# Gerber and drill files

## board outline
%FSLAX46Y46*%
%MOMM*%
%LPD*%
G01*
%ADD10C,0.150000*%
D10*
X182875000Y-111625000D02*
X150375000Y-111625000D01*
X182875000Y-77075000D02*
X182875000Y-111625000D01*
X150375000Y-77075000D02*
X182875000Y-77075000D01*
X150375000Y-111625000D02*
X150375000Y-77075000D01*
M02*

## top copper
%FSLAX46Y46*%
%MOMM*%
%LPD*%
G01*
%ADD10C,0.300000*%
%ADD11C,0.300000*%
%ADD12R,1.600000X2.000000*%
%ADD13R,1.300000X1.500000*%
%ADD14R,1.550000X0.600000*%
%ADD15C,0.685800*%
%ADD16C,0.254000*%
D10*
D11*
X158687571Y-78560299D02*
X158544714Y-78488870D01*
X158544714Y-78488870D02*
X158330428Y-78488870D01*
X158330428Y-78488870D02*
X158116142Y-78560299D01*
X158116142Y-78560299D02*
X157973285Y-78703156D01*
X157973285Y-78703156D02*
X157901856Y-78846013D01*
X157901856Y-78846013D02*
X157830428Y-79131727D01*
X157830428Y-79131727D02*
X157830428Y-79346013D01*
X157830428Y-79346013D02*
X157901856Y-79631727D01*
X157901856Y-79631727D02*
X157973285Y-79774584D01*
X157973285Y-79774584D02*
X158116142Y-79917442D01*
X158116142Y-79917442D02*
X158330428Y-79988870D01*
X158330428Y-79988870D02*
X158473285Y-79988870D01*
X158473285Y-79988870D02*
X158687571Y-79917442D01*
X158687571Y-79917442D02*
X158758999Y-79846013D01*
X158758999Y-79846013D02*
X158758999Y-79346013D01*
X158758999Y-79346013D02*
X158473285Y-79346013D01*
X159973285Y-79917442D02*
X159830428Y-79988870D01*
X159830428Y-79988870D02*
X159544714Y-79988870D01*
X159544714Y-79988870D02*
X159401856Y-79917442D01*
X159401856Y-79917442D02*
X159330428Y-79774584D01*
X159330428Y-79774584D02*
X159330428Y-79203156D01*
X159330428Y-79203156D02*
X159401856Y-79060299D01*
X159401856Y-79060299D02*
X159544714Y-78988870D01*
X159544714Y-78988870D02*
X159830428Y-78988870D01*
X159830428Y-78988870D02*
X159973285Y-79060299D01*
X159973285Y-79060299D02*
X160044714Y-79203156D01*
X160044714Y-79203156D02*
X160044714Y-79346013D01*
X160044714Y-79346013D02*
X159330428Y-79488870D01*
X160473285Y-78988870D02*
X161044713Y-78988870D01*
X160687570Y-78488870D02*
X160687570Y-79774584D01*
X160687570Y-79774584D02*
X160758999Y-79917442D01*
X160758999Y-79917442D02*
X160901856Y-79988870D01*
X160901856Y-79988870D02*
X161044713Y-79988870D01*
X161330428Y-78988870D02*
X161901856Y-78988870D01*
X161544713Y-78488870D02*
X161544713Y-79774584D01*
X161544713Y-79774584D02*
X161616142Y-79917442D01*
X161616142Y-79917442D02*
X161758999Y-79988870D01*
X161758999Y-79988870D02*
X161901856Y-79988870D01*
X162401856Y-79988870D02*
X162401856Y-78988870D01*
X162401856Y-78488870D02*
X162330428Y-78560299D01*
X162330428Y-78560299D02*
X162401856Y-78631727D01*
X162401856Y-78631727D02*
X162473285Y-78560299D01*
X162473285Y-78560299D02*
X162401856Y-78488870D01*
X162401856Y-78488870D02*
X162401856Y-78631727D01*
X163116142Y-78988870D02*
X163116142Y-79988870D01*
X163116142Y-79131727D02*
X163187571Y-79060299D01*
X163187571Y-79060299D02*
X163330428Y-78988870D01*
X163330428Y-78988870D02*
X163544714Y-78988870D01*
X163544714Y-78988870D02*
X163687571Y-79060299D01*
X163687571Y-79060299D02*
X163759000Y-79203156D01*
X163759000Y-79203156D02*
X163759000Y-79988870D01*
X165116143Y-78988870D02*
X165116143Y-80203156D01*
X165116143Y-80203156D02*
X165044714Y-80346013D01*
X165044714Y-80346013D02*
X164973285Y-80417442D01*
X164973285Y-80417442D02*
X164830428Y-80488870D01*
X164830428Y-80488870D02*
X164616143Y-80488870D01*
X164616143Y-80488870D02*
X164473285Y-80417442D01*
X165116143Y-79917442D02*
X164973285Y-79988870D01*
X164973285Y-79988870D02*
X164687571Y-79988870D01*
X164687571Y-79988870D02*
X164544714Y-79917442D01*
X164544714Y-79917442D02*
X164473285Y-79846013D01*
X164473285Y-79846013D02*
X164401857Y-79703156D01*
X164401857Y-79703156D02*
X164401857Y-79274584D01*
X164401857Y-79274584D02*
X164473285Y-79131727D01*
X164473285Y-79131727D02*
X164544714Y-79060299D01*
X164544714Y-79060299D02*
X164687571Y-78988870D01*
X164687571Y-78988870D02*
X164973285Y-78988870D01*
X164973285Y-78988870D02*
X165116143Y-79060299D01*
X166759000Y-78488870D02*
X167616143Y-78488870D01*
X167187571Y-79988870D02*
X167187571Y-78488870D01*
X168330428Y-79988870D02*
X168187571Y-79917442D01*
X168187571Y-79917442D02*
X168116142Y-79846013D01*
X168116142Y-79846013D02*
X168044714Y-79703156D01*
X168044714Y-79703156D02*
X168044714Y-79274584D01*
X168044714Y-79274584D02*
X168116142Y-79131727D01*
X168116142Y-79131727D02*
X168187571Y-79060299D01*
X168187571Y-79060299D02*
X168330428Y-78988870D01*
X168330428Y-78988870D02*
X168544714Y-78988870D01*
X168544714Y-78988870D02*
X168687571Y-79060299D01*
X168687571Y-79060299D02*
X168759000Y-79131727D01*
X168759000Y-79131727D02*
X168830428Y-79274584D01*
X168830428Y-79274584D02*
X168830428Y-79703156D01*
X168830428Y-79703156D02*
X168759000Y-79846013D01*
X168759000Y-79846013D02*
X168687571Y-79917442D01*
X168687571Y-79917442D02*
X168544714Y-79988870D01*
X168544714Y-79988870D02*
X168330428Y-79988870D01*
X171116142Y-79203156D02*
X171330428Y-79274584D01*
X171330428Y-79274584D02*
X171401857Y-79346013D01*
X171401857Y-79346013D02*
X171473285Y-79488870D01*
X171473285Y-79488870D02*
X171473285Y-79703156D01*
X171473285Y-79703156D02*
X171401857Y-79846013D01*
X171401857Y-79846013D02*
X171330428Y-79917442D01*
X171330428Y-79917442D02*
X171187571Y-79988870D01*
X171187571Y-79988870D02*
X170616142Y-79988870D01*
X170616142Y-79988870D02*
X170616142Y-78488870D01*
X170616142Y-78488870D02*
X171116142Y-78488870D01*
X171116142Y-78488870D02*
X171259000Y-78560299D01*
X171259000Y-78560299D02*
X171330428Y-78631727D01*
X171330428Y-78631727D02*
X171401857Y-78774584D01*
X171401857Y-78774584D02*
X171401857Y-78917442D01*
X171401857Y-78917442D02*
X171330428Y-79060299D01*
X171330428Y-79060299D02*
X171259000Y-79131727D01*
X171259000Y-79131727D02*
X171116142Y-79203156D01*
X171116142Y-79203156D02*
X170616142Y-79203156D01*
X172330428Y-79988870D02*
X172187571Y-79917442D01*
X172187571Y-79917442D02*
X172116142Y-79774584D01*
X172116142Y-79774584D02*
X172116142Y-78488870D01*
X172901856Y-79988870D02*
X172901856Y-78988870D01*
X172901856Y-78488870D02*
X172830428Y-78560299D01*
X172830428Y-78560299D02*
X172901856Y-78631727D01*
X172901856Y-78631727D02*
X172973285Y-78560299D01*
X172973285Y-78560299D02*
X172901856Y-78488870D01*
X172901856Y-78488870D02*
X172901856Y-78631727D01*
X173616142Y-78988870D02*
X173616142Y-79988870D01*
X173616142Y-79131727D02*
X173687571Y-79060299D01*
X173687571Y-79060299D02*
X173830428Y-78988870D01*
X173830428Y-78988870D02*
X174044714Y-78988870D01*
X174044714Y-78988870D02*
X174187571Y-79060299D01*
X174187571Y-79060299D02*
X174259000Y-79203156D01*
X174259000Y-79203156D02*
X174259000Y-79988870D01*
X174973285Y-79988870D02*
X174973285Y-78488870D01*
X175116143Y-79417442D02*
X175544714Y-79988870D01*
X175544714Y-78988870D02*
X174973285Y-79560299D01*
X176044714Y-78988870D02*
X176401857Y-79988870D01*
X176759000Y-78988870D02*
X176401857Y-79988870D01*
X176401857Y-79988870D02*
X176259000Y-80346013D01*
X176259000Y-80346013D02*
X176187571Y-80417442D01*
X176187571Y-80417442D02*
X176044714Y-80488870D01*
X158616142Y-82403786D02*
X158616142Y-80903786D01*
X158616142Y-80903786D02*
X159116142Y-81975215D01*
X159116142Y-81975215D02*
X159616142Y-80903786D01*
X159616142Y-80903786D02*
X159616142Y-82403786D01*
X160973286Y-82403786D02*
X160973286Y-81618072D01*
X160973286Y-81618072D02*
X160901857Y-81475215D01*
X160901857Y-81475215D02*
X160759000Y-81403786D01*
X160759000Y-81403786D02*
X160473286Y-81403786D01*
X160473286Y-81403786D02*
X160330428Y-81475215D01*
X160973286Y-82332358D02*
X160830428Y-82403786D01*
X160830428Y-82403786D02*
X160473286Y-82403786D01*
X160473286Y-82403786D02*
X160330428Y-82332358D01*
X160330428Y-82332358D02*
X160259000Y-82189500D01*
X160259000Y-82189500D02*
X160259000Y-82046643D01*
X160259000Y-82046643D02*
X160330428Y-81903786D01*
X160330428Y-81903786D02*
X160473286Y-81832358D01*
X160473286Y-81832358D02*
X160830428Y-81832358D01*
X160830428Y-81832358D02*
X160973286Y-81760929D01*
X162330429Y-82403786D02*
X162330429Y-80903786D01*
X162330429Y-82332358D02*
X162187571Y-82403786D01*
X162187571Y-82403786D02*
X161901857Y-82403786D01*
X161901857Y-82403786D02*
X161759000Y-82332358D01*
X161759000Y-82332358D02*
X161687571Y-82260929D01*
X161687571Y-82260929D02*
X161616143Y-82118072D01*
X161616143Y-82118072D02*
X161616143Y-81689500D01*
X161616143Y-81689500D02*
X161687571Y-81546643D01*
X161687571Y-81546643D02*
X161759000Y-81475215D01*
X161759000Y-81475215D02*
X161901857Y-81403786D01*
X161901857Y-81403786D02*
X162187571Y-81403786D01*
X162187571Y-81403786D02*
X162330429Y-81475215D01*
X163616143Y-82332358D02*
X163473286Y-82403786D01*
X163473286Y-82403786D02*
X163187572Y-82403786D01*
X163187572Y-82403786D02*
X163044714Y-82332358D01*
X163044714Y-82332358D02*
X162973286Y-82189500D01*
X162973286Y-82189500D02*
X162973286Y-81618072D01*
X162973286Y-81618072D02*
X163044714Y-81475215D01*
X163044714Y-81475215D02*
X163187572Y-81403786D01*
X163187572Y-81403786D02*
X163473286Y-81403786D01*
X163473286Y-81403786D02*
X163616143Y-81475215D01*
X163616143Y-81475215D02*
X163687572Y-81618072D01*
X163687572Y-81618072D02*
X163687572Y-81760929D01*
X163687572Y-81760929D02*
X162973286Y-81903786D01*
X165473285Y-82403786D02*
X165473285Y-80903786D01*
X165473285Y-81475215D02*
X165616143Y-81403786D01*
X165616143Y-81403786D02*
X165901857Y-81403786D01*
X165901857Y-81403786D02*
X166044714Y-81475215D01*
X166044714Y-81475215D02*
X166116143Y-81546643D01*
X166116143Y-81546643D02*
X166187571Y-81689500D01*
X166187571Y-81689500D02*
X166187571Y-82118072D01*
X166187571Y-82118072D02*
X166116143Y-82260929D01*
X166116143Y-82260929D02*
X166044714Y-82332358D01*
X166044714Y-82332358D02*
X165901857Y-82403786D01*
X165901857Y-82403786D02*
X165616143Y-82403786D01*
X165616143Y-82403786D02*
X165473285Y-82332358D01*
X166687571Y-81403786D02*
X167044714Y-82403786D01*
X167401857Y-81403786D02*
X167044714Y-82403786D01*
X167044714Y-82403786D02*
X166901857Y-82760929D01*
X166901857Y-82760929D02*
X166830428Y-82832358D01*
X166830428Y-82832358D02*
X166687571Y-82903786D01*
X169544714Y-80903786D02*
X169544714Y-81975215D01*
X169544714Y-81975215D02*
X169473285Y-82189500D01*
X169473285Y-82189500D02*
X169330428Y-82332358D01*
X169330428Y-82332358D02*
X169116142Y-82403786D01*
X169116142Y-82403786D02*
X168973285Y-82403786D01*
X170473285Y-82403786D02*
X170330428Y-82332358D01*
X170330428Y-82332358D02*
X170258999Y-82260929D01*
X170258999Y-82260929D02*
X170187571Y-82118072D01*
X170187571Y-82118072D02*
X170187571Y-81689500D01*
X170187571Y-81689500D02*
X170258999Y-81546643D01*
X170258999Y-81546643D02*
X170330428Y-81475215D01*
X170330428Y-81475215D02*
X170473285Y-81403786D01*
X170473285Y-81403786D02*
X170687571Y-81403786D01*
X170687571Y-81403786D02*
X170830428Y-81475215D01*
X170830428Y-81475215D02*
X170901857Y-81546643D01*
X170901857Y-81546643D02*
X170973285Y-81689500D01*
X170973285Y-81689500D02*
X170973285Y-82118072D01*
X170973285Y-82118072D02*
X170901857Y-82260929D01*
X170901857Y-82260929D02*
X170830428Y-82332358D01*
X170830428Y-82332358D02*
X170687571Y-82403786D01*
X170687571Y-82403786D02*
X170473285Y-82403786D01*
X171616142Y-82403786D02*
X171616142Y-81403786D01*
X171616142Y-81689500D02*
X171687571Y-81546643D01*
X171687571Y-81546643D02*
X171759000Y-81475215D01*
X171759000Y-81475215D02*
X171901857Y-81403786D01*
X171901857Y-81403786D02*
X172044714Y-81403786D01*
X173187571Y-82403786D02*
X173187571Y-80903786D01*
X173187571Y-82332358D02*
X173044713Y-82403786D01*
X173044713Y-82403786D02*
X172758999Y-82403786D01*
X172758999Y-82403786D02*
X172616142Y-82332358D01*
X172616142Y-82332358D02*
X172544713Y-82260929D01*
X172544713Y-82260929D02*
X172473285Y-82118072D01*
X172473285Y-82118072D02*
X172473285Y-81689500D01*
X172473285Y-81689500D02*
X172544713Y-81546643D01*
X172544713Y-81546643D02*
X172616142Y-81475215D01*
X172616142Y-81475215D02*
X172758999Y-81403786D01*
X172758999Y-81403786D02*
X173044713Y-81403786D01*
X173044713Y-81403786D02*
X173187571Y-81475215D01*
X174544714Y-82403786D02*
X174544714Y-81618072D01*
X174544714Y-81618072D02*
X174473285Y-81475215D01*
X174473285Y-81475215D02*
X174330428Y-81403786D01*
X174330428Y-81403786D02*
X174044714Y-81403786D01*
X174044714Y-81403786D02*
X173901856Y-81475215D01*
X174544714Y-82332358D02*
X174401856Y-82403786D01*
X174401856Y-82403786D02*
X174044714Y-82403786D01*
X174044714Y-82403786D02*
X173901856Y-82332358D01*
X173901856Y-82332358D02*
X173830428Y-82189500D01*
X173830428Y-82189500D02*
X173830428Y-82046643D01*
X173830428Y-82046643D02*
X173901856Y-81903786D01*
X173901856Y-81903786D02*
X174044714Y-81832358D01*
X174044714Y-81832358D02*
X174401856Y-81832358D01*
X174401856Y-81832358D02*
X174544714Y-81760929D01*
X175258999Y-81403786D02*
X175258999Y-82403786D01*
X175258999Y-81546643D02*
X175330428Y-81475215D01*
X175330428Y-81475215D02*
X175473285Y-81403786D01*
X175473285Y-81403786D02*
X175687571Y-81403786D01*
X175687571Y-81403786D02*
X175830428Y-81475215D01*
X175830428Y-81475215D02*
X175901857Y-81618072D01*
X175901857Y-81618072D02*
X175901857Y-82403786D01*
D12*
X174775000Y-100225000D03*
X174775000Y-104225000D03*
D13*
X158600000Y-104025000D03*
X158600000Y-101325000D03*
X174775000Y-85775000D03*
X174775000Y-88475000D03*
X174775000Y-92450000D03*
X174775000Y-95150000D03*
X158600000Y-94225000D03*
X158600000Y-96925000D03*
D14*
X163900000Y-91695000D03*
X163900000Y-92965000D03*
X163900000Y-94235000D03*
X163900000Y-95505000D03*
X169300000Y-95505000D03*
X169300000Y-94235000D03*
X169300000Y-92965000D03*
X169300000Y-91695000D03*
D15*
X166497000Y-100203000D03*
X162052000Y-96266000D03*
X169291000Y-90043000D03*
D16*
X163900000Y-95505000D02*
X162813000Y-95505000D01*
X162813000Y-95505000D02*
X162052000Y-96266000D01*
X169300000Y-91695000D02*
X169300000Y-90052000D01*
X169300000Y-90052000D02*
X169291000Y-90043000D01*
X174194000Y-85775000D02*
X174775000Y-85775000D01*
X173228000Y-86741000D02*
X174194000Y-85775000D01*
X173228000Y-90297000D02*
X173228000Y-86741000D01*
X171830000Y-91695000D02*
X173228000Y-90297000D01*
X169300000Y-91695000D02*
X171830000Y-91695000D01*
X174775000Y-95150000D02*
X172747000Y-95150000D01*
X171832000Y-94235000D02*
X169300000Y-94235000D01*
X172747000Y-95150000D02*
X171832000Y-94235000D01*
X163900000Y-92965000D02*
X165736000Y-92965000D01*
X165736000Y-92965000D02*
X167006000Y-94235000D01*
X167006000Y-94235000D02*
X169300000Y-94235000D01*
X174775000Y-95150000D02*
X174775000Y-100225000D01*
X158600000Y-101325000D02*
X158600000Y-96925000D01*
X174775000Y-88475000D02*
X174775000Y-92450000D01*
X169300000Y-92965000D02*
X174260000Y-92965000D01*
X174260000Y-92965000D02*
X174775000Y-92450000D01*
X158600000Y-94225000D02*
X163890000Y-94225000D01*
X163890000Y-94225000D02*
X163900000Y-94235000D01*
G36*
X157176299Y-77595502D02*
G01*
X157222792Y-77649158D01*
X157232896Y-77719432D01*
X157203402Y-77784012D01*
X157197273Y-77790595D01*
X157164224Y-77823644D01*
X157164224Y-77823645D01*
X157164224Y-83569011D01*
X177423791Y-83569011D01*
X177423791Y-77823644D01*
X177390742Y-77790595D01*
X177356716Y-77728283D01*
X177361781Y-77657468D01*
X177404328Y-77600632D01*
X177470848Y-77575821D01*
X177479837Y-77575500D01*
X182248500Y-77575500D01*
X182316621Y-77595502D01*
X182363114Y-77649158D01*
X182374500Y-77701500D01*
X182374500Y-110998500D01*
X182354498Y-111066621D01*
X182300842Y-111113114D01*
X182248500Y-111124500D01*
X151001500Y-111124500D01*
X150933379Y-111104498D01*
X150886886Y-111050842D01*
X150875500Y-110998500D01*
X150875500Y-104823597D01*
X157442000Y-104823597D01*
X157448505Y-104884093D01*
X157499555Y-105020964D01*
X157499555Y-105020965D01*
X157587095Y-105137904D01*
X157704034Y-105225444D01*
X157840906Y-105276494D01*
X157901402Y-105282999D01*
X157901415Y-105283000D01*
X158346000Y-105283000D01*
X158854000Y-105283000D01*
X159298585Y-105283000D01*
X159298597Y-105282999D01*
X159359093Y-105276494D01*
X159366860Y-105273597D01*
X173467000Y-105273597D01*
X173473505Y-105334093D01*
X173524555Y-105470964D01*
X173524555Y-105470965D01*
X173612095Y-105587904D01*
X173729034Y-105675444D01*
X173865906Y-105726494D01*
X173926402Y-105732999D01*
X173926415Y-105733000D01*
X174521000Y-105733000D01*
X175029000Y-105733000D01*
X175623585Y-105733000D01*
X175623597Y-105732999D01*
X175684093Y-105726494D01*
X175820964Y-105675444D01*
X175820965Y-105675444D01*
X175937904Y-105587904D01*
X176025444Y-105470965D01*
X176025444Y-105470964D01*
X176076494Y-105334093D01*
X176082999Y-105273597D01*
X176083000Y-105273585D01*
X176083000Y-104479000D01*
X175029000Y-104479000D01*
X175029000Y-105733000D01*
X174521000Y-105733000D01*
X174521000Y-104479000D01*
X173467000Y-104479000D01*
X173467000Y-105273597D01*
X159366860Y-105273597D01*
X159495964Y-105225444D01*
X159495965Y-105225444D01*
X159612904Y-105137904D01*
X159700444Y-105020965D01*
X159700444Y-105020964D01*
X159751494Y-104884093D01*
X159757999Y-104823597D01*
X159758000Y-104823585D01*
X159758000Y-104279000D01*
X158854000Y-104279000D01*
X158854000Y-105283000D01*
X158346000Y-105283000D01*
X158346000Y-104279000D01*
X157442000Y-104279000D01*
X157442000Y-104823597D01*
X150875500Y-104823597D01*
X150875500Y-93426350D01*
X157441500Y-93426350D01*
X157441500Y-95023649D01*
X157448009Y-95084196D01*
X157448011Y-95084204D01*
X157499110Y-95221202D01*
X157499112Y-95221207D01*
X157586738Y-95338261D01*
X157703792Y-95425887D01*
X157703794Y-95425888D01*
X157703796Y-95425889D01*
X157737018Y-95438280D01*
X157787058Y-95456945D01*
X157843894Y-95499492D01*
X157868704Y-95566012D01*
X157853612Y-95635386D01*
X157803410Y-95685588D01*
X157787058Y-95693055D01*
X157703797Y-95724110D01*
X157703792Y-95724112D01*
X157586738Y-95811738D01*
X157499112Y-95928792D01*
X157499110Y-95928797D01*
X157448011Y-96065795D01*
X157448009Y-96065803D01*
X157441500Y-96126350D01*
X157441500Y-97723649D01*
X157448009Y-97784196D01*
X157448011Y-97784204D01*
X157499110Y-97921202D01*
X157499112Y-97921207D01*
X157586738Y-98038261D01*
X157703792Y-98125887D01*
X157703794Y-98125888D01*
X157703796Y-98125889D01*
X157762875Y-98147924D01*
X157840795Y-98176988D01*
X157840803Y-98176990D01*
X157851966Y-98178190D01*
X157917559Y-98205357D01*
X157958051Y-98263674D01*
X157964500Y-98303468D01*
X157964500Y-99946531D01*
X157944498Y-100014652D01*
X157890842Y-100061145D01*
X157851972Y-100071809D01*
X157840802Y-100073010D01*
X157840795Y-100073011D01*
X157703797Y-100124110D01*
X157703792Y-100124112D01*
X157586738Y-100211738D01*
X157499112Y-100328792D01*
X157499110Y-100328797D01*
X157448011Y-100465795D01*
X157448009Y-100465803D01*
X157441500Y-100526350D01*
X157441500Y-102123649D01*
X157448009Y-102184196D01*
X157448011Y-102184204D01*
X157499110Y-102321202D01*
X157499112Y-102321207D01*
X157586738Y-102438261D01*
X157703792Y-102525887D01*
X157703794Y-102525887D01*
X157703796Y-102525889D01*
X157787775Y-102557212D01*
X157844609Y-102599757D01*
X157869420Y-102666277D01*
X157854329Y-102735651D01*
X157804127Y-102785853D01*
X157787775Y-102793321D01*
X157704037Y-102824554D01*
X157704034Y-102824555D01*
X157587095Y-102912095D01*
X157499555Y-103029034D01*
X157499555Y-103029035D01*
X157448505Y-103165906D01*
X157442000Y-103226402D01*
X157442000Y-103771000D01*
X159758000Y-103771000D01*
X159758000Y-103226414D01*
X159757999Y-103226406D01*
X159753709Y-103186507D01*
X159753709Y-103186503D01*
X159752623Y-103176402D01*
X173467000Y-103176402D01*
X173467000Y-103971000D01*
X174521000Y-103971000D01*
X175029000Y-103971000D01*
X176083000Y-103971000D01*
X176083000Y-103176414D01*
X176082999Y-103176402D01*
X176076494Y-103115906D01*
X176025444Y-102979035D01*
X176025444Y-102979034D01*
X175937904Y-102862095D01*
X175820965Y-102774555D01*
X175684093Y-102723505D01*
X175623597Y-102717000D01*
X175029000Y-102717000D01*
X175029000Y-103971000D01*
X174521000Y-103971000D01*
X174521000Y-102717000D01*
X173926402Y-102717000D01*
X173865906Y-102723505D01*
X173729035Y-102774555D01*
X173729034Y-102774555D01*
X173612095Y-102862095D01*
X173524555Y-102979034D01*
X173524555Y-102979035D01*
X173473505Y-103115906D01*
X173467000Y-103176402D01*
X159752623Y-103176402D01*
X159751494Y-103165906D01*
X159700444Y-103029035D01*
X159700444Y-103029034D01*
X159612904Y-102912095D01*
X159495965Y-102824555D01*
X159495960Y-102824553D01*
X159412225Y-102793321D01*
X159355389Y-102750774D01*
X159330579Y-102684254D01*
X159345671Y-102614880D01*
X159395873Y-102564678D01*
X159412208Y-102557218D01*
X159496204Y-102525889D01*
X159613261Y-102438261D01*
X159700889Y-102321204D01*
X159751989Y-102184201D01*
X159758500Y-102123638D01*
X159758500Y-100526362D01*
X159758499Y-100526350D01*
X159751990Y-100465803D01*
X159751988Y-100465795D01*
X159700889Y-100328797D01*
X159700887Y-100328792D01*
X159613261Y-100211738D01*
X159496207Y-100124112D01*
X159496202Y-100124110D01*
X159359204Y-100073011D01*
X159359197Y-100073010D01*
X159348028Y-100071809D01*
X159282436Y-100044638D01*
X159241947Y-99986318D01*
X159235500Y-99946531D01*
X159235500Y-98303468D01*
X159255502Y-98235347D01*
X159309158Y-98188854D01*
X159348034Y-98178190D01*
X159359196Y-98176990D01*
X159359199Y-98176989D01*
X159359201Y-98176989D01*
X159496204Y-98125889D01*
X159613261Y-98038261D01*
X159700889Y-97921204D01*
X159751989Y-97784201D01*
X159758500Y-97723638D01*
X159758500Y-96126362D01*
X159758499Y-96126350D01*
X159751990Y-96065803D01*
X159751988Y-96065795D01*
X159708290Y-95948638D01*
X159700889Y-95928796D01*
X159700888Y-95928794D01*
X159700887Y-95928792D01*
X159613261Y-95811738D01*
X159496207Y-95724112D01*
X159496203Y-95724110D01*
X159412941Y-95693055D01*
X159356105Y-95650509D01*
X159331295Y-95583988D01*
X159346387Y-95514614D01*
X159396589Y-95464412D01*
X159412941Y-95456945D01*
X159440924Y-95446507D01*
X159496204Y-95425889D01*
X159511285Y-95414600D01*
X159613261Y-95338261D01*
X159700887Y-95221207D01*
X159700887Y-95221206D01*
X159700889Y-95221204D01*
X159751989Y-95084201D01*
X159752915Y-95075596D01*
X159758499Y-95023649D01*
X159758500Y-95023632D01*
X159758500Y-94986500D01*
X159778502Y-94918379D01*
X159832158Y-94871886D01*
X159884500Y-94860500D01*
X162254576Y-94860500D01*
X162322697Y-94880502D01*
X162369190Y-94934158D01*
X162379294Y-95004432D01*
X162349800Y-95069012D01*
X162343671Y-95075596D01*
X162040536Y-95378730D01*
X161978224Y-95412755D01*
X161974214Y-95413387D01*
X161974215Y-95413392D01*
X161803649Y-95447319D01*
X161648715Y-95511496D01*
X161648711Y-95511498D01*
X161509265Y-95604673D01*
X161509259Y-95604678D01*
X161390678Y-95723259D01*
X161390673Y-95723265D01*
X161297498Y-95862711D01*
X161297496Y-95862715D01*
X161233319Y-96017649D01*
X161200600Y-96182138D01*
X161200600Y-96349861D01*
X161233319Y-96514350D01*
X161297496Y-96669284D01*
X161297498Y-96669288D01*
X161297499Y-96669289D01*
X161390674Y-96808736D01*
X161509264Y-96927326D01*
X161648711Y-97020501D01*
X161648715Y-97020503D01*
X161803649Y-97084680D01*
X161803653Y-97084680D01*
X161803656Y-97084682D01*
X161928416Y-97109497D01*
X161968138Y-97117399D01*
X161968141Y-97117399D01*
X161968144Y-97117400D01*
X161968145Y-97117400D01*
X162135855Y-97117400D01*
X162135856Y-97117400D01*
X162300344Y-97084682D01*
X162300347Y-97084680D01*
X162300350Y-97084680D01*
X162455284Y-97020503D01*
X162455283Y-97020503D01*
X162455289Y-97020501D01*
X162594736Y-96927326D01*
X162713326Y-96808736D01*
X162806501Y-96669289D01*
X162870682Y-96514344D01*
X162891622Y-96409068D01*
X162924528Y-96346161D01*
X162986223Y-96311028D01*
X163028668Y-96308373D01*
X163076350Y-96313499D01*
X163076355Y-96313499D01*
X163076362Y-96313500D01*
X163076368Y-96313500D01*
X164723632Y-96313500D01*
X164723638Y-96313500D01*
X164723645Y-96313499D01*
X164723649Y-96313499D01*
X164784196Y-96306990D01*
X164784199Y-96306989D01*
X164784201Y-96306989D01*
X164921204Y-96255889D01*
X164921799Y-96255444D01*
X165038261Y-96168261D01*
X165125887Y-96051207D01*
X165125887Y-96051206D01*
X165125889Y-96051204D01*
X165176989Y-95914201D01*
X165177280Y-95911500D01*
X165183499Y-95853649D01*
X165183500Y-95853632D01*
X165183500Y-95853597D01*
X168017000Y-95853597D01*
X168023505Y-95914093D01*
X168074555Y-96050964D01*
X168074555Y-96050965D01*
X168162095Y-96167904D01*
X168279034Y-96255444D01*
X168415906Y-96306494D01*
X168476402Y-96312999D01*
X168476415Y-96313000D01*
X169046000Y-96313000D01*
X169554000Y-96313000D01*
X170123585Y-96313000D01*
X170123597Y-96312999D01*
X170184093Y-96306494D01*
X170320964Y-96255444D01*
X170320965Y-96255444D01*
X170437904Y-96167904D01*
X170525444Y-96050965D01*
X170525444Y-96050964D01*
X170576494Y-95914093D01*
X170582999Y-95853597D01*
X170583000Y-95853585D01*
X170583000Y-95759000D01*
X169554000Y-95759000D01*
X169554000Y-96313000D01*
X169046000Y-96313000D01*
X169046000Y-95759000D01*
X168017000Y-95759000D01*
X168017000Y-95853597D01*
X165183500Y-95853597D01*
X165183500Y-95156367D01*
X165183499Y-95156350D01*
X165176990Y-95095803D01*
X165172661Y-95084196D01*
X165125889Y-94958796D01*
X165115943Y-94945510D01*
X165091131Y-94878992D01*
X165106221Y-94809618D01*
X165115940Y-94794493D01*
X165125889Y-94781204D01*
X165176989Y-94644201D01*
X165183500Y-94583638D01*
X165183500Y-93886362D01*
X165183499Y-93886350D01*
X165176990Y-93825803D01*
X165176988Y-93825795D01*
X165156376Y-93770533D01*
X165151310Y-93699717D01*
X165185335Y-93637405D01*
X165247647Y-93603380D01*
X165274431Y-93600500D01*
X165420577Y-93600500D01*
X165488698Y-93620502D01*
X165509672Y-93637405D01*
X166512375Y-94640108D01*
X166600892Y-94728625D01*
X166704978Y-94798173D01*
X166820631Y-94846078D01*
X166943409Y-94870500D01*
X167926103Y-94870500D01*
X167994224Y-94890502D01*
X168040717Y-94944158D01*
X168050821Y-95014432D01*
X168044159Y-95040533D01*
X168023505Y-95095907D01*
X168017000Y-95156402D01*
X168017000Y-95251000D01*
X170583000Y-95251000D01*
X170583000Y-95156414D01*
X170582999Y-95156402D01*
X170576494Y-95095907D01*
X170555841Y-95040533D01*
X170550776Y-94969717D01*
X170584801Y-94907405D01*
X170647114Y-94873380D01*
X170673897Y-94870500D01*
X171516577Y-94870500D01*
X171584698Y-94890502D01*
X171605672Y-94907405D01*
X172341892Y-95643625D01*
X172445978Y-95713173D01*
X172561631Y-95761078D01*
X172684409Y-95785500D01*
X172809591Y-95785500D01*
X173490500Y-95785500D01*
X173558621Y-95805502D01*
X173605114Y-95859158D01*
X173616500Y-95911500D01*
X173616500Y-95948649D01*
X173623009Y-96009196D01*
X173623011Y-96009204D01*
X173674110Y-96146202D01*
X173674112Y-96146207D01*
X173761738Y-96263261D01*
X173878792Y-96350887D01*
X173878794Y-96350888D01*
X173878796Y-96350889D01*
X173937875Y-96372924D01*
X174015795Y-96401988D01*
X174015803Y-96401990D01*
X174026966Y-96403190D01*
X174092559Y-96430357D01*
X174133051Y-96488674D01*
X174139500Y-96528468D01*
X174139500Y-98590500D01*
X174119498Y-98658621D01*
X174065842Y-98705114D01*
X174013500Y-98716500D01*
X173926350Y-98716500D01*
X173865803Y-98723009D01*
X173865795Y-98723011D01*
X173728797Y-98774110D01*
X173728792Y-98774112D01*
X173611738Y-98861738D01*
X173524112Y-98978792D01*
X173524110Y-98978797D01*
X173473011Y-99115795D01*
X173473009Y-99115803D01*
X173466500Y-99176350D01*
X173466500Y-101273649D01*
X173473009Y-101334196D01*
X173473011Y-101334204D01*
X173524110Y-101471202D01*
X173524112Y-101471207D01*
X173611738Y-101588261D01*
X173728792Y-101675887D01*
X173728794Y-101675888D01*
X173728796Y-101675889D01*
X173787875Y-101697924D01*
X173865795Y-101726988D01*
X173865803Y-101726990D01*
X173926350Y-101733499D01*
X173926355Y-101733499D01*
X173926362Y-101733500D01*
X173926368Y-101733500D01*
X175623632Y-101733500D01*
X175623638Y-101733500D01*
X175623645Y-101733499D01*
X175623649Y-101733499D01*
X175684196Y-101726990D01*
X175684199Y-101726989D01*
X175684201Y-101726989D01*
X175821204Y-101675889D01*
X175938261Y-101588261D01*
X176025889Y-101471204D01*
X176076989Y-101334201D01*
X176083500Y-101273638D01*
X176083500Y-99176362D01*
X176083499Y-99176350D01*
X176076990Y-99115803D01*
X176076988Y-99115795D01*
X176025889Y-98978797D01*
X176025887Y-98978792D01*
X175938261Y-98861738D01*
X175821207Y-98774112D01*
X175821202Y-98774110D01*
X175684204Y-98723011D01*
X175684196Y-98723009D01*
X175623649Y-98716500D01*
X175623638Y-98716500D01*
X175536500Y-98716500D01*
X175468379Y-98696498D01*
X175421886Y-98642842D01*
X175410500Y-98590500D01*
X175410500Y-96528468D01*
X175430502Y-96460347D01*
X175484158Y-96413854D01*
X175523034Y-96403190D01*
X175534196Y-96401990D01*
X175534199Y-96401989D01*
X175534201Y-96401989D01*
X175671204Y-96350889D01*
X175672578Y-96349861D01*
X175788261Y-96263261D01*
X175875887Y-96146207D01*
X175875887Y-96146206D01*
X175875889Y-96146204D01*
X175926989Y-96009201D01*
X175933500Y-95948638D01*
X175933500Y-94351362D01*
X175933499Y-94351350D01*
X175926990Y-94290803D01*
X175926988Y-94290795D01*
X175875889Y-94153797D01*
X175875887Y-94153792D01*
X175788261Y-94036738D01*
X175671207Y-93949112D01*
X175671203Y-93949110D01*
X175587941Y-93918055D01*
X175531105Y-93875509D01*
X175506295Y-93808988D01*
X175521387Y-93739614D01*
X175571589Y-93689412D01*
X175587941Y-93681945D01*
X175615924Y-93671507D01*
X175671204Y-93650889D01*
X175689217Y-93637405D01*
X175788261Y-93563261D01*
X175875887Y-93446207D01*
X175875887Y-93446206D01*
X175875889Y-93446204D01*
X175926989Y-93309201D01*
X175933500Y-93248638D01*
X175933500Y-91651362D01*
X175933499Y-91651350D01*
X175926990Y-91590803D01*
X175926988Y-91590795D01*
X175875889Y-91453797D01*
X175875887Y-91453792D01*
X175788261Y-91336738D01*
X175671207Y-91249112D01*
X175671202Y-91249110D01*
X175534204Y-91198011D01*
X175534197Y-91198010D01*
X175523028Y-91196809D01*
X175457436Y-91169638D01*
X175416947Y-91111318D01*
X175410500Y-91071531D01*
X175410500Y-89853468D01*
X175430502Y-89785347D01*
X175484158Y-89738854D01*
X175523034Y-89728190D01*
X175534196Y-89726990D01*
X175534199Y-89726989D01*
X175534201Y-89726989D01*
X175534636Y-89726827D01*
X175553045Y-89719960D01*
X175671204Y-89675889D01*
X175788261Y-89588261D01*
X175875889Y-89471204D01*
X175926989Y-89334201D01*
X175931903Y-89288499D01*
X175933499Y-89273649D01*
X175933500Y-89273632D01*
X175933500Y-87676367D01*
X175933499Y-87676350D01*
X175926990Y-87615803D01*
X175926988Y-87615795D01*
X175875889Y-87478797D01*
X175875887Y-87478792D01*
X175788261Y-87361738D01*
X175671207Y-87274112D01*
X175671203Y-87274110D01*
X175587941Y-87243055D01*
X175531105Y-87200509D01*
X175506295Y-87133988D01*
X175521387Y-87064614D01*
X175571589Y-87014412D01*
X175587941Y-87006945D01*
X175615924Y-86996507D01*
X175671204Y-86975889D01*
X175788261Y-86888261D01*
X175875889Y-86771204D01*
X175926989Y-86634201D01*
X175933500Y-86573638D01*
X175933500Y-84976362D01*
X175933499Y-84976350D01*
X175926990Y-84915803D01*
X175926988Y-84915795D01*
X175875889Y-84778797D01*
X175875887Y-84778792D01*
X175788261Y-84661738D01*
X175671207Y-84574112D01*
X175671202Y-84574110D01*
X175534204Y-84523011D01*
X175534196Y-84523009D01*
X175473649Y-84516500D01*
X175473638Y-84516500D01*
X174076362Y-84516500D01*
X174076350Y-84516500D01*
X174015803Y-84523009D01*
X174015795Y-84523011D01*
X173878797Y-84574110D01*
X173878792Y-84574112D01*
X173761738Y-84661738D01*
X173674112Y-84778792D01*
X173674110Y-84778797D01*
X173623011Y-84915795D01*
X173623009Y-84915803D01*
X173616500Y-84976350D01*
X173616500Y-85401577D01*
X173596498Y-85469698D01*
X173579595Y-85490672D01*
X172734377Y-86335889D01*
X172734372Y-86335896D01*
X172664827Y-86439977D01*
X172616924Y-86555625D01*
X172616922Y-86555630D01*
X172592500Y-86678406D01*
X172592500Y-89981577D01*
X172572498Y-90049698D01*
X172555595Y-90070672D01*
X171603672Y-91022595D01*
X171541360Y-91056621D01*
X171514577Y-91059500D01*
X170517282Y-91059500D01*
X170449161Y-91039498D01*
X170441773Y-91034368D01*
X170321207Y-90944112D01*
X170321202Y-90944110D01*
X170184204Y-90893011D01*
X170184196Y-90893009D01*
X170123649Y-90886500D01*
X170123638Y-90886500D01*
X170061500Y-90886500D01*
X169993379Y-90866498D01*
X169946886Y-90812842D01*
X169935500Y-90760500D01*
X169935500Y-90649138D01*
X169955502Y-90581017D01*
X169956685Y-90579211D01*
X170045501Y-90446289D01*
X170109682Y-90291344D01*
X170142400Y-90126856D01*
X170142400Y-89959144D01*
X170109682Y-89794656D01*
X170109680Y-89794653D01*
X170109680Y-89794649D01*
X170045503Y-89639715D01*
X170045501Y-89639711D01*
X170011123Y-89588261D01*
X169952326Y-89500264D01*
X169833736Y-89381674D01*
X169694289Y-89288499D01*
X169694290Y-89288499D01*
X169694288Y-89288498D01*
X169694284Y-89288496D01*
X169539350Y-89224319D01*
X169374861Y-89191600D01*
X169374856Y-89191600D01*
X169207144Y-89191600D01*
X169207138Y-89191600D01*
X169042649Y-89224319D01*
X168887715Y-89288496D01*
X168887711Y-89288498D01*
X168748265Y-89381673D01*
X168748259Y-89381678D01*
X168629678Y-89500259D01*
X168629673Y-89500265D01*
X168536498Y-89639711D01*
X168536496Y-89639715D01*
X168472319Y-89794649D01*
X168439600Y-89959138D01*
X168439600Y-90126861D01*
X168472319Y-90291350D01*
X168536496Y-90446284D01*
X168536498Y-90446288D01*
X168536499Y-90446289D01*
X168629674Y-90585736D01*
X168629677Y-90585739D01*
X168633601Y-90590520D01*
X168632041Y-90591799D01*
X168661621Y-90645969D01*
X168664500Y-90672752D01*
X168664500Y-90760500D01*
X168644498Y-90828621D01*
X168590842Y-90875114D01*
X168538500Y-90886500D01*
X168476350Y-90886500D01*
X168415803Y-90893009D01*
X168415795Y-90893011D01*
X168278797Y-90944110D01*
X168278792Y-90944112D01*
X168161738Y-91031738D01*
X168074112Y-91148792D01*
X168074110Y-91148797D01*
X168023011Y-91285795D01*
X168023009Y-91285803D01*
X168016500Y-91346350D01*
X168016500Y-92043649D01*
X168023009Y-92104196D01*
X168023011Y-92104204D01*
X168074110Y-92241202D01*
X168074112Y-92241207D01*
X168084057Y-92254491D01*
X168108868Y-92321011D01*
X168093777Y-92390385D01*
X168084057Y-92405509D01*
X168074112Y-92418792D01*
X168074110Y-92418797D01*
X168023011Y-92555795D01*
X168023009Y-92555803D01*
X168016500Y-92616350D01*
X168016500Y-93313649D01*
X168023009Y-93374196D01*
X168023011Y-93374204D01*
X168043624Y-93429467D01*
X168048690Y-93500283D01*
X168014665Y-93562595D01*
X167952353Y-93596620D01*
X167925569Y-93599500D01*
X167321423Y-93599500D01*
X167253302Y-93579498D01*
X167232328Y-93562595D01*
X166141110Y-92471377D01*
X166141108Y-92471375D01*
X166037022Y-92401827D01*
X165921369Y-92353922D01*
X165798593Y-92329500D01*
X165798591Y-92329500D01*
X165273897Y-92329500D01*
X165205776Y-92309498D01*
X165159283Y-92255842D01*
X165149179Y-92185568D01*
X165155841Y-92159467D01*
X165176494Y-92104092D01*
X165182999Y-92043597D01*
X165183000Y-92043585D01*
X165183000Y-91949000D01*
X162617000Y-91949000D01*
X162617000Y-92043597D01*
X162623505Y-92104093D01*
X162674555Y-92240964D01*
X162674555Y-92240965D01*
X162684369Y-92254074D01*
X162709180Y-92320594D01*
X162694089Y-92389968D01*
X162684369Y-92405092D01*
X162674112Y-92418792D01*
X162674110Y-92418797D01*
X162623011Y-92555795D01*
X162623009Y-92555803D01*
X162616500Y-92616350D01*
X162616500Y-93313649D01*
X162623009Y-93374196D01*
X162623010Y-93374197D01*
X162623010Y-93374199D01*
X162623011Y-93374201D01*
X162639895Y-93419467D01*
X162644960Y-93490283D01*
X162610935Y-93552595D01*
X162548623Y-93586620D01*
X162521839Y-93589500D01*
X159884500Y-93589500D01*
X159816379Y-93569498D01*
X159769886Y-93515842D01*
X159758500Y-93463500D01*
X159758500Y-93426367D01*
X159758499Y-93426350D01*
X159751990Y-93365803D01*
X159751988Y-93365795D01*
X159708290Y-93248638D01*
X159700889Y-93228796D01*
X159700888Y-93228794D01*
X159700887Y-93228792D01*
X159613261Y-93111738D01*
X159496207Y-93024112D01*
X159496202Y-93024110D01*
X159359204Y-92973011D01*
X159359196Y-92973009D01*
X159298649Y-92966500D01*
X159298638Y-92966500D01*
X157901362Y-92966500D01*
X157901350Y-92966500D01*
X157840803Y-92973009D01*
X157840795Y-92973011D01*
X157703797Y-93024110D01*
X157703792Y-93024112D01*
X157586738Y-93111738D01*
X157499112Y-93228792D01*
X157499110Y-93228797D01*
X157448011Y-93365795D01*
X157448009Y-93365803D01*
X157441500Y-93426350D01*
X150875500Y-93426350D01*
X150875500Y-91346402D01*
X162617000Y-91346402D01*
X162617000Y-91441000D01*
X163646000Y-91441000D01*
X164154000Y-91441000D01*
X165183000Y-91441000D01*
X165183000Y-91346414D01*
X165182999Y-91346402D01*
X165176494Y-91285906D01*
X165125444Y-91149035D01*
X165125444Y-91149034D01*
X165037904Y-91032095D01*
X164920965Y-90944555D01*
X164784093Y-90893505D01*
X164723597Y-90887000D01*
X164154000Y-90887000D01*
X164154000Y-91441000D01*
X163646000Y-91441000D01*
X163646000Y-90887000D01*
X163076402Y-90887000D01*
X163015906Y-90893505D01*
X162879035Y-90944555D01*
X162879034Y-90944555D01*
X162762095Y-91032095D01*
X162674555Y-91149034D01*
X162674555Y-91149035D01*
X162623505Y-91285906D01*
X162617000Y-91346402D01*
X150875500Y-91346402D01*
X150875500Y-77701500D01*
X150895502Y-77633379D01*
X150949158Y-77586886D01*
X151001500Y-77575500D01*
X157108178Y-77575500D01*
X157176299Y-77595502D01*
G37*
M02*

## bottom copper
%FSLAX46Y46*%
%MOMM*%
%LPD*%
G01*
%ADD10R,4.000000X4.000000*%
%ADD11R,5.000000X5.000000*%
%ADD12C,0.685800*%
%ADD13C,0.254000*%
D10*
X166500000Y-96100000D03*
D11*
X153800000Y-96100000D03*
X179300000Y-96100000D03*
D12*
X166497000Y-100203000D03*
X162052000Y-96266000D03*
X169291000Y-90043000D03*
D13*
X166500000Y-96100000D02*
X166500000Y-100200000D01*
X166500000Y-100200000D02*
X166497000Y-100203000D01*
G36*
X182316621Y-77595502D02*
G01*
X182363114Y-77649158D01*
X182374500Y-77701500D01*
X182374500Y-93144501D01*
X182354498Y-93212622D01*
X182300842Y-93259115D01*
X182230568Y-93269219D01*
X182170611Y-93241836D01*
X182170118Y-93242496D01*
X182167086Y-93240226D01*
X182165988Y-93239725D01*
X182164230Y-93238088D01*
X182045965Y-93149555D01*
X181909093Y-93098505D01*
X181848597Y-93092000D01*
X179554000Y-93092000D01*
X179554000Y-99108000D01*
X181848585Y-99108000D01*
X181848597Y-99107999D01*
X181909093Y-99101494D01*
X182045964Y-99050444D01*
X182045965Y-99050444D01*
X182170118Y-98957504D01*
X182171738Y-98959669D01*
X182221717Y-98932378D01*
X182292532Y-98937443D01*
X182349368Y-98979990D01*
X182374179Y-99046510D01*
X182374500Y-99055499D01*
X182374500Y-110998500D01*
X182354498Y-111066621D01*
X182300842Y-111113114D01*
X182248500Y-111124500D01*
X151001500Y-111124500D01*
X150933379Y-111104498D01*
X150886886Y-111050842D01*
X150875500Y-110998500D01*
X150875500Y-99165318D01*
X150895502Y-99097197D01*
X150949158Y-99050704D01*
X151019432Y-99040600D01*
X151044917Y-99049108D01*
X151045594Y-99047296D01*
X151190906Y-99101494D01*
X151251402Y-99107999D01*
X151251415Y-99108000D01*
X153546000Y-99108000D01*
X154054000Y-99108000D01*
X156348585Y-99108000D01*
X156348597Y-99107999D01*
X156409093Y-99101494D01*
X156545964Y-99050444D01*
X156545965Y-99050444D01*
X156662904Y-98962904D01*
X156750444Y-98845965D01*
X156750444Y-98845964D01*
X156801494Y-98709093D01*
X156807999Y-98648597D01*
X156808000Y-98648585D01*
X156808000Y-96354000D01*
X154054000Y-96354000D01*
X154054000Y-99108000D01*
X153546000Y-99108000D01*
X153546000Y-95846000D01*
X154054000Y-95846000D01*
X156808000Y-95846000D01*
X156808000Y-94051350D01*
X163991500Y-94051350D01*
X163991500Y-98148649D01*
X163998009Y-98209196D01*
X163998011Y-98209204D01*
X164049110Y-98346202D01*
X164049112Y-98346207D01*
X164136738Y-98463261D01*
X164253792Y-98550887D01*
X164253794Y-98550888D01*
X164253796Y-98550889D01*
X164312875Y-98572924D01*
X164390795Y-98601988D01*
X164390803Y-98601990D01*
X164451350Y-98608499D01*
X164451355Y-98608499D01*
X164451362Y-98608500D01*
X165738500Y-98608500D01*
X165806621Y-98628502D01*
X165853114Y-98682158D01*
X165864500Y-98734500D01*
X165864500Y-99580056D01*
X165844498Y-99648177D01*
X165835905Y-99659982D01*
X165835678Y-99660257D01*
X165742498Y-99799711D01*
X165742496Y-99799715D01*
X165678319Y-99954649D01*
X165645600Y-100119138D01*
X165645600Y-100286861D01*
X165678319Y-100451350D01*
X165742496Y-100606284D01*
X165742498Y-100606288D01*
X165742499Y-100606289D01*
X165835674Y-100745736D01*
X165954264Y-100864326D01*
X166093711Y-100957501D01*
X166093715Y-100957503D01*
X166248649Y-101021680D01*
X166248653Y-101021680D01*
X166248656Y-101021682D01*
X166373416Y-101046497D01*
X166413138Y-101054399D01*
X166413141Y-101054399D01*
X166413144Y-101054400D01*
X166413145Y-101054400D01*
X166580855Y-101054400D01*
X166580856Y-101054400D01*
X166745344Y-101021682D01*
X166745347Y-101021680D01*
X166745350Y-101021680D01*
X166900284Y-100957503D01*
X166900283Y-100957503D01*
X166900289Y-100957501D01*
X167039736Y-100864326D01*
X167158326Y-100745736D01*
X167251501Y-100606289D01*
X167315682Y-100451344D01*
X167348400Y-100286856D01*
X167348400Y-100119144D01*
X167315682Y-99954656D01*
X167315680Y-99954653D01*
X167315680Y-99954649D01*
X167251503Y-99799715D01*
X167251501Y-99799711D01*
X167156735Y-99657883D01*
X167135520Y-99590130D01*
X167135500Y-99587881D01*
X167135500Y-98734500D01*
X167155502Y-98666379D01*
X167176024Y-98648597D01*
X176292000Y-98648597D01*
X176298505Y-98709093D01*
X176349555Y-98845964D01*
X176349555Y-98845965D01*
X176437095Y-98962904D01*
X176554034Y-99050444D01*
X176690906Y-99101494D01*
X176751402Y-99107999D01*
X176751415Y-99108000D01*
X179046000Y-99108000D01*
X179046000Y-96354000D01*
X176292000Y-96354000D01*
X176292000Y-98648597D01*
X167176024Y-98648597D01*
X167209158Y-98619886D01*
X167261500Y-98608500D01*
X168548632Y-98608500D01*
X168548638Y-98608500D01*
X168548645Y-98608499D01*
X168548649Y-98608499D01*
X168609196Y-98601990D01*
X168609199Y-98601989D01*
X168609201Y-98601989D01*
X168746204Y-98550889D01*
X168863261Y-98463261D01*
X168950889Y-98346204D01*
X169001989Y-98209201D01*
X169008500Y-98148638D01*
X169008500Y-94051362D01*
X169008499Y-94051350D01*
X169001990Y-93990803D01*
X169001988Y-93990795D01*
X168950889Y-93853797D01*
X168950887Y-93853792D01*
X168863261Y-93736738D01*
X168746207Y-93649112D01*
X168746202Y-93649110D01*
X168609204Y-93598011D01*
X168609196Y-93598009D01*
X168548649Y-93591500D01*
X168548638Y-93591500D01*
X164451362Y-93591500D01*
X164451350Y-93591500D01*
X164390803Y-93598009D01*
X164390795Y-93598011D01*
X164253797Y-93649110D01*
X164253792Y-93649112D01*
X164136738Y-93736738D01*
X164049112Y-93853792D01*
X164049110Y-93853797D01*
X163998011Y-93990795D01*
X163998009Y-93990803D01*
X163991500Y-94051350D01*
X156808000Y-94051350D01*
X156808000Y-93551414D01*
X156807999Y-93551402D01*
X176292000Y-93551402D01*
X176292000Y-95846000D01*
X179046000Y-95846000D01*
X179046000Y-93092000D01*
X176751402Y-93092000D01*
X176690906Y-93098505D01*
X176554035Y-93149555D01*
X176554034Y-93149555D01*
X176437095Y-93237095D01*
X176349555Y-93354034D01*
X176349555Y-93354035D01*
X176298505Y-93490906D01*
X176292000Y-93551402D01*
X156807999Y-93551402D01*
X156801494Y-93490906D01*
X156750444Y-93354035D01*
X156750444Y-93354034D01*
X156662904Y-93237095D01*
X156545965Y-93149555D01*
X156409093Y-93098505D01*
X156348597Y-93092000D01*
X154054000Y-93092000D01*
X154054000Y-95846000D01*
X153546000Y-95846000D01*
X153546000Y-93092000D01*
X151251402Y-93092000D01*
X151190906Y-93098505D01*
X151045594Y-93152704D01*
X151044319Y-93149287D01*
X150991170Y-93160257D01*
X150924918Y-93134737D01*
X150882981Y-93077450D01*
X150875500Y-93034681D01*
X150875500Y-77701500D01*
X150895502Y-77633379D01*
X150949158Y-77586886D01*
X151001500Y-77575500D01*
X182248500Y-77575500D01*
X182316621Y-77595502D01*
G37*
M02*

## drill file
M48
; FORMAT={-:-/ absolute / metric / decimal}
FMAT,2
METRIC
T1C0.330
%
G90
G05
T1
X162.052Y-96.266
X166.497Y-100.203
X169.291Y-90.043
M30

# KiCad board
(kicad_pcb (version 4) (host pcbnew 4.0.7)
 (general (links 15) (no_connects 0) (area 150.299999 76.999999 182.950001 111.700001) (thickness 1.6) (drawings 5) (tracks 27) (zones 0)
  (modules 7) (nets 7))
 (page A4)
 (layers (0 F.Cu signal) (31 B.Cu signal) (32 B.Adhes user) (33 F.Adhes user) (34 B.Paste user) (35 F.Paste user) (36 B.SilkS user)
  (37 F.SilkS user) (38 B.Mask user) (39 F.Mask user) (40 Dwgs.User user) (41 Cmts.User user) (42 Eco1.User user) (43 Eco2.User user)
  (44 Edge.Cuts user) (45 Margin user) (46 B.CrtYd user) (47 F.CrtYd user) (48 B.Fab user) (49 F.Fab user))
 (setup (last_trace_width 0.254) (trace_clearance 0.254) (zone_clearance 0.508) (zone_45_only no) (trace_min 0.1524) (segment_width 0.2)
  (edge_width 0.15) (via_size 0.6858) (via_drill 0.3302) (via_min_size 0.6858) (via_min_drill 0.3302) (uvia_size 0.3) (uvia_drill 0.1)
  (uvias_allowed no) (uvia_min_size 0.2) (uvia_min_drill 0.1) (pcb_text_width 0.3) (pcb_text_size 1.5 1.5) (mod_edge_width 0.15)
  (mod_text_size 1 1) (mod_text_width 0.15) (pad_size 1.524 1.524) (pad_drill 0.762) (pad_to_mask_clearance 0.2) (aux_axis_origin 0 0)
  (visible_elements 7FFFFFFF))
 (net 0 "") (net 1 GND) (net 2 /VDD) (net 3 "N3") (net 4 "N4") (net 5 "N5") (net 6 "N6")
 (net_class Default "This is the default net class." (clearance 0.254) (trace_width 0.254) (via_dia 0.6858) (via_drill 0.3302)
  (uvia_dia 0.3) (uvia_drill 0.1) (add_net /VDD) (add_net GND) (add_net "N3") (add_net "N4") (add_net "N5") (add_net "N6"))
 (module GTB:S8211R (layer B.Cu) (at 166.5 96.1)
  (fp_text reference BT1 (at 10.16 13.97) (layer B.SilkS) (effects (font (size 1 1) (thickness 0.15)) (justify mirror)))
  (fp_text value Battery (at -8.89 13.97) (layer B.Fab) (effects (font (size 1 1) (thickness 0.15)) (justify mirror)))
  (pad 2 smd rect (at 0 0) (size 4 4) (layers B.Cu B.Paste B.Mask) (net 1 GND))
  (pad 1 smd rect (at -12.7 0) (size 5 5) (layers B.Cu B.Paste B.Mask) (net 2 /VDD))
  (pad 1 smd rect (at 12.8 0) (size 5 5) (layers B.Cu B.Paste B.Mask) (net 2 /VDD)))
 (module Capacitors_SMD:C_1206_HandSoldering (layer F.Cu) (at 174.775 102.225 270)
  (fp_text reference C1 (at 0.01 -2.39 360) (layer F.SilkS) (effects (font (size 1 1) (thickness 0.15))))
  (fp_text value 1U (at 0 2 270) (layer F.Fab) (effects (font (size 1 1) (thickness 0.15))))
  (pad 1 smd rect (at -2 0 270) (size 2 1.6) (layers F.Cu F.Paste F.Mask) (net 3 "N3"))
  (pad 2 smd rect (at 2 0 270) (size 2 1.6) (layers F.Cu F.Paste F.Mask) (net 1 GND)))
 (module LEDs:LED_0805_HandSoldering (layer F.Cu) (at 158.6 102.675 90)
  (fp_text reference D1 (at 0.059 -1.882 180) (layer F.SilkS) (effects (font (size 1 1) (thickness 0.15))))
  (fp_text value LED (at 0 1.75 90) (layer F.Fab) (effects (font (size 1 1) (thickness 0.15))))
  (pad 1 smd rect (at -1.35 0 90) (size 1.5 1.3) (layers F.Cu F.Paste F.Mask) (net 1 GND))
  (pad 2 smd rect (at 1.35 0 90) (size 1.5 1.3) (layers F.Cu F.Paste F.Mask) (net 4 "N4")))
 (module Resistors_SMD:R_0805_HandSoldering (layer F.Cu) (at 174.775 87.125 270)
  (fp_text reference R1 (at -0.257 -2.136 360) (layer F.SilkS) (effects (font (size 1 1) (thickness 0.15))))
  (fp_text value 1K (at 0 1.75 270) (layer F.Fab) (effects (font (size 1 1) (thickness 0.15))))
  (pad 1 smd rect (at -1.35 0 270) (size 1.5 1.3) (layers F.Cu F.Paste F.Mask) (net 2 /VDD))
  (pad 2 smd rect (at 1.35 0 270) (size 1.5 1.3) (layers F.Cu F.Paste F.Mask) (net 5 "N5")))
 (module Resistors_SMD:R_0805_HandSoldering (layer F.Cu) (at 174.775 93.8 270)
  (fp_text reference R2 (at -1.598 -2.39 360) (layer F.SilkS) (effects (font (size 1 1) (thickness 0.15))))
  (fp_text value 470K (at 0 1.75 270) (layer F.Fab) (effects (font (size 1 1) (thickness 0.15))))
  (pad 1 smd rect (at -1.35 0 270) (size 1.5 1.3) (layers F.Cu F.Paste F.Mask) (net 5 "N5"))
  (pad 2 smd rect (at 1.35 0 270) (size 1.5 1.3) (layers F.Cu F.Paste F.Mask) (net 3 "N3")))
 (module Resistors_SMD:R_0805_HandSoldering (layer F.Cu) (at 158.6 95.575 270)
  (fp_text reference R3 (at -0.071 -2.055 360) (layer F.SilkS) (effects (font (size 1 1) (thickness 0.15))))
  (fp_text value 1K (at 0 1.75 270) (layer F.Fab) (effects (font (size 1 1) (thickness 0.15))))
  (pad 1 smd rect (at -1.35 0 270) (size 1.5 1.3) (layers F.Cu F.Paste F.Mask) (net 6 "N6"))
  (pad 2 smd rect (at 1.35 0 270) (size 1.5 1.3) (layers F.Cu F.Paste F.Mask) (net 4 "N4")))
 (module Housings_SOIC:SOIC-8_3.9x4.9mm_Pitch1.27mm (layer F.Cu) (at 166.6 93.6)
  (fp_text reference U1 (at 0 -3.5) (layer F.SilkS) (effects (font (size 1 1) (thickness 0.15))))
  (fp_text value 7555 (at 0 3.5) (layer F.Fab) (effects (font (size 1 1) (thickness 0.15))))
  (pad 1 smd rect (at -2.7 -1.905) (size 1.55 0.6) (layers F.Cu F.Paste F.Mask) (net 1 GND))
  (pad 2 smd rect (at -2.7 -0.635) (size 1.55 0.6) (layers F.Cu F.Paste F.Mask) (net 3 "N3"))
  (pad 3 smd rect (at -2.7 0.635) (size 1.55 0.6) (layers F.Cu F.Paste F.Mask) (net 6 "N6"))
  (pad 4 smd rect (at -2.7 1.905) (size 1.55 0.6) (layers F.Cu F.Paste F.Mask) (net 2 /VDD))
  (pad 5 smd rect (at 2.7 1.905) (size 1.55 0.6) (layers F.Cu F.Paste F.Mask) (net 1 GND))
  (pad 6 smd rect (at 2.7 0.635) (size 1.55 0.6) (layers F.Cu F.Paste F.Mask) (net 3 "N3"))
  (pad 7 smd rect (at 2.7 -0.635) (size 1.55 0.6) (layers F.Cu F.Paste F.Mask) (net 5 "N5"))
  (pad 8 smd rect (at 2.7 -1.905) (size 1.55 0.6) (layers F.Cu F.Paste F.Mask) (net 2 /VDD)))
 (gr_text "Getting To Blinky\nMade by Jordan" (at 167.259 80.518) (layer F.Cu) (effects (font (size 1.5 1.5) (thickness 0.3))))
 (gr_line (start 182.875 111.625) (end 150.375 111.625) (angle 90) (layer Edge.Cuts) (width 0.15))
 (gr_line (start 182.875 77.075) (end 182.875 111.625) (angle 90) (layer Edge.Cuts) (width 0.15))
 (gr_line (start 150.375 77.075) (end 182.875 77.075) (angle 90) (layer Edge.Cuts) (width 0.15))
 (gr_line (start 150.375 111.625) (end 150.375 77.075) (angle 90) (layer Edge.Cuts) (width 0.15))
 (segment (start 166.5 96.1) (end 166.5 100.2) (width 0.254) (layer B.Cu) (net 1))
 (via (at 166.497 100.203) (size 0.6858) (drill 0.3302) (layers F.Cu B.Cu) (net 1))
 (segment (start 166.5 100.2) (end 166.497 100.203) (width 0.254) (layer B.Cu) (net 1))
 (segment (start 163.9 95.505) (end 162.813 95.505) (width 0.254) (layer F.Cu) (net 2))
 (via (at 162.052 96.266) (size 0.6858) (drill 0.3302) (layers F.Cu B.Cu) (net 2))
 (segment (start 162.813 95.505) (end 162.052 96.266) (width 0.254) (layer F.Cu) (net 2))
 (segment (start 169.3 91.695) (end 169.3 90.052) (width 0.254) (layer F.Cu) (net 2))
 (via (at 169.291 90.043) (size 0.6858) (drill 0.3302) (layers F.Cu B.Cu) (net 2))
 (segment (start 169.3 90.052) (end 169.291 90.043) (width 0.254) (layer F.Cu) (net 2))
 (segment (start 174.194 85.775) (end 174.775 85.775) (width 0.254) (layer F.Cu) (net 2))
 (segment (start 173.228 86.741) (end 174.194 85.775) (width 0.254) (layer F.Cu) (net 2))
 (segment (start 173.228 90.297) (end 173.228 86.741) (width 0.254) (layer F.Cu) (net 2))
 (segment (start 171.83 91.695) (end 173.228 90.297) (width 0.254) (layer F.Cu) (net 2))
 (segment (start 169.3 91.695) (end 171.83 91.695) (width 0.254) (layer F.Cu) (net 2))
 (segment (start 174.775 95.15) (end 172.747 95.15) (width 0.254) (layer F.Cu) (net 3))
 (segment (start 171.832 94.235) (end 169.3 94.235) (width 0.254) (layer F.Cu) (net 3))
 (segment (start 172.747 95.15) (end 171.832 94.235) (width 0.254) (layer F.Cu) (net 3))
 (segment (start 163.9 92.965) (end 165.736 92.965) (width 0.254) (layer F.Cu) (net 3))
 (segment (start 165.736 92.965) (end 167.006 94.235) (width 0.254) (layer F.Cu) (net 3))
 (segment (start 167.006 94.235) (end 169.3 94.235) (width 0.254) (layer F.Cu) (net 3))
 (segment (start 174.775 95.15) (end 174.775 100.225) (width 0.254) (layer F.Cu) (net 3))
 (segment (start 158.6 101.325) (end 158.6 96.925) (width 0.254) (layer F.Cu) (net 4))
 (segment (start 174.775 88.475) (end 174.775 92.45) (width 0.254) (layer F.Cu) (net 5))
 (segment (start 169.3 92.965) (end 174.26 92.965) (width 0.254) (layer F.Cu) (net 5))
 (segment (start 174.26 92.965) (end 174.775 92.45) (width 0.254) (layer F.Cu) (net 5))
 (segment (start 158.6 94.225) (end 163.89 94.225) (width 0.254) (layer F.Cu) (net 6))
 (segment (start 163.89 94.225) (end 163.9 94.235) (width 0.254) (layer F.Cu) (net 6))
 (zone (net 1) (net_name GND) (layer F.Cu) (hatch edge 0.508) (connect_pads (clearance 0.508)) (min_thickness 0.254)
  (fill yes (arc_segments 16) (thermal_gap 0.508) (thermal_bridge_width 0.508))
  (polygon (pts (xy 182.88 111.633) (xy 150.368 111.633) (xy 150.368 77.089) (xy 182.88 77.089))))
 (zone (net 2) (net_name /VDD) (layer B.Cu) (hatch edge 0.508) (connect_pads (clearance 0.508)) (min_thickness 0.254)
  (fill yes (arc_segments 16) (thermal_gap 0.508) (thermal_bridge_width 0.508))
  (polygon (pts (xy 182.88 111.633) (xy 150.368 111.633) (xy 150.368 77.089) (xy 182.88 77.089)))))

